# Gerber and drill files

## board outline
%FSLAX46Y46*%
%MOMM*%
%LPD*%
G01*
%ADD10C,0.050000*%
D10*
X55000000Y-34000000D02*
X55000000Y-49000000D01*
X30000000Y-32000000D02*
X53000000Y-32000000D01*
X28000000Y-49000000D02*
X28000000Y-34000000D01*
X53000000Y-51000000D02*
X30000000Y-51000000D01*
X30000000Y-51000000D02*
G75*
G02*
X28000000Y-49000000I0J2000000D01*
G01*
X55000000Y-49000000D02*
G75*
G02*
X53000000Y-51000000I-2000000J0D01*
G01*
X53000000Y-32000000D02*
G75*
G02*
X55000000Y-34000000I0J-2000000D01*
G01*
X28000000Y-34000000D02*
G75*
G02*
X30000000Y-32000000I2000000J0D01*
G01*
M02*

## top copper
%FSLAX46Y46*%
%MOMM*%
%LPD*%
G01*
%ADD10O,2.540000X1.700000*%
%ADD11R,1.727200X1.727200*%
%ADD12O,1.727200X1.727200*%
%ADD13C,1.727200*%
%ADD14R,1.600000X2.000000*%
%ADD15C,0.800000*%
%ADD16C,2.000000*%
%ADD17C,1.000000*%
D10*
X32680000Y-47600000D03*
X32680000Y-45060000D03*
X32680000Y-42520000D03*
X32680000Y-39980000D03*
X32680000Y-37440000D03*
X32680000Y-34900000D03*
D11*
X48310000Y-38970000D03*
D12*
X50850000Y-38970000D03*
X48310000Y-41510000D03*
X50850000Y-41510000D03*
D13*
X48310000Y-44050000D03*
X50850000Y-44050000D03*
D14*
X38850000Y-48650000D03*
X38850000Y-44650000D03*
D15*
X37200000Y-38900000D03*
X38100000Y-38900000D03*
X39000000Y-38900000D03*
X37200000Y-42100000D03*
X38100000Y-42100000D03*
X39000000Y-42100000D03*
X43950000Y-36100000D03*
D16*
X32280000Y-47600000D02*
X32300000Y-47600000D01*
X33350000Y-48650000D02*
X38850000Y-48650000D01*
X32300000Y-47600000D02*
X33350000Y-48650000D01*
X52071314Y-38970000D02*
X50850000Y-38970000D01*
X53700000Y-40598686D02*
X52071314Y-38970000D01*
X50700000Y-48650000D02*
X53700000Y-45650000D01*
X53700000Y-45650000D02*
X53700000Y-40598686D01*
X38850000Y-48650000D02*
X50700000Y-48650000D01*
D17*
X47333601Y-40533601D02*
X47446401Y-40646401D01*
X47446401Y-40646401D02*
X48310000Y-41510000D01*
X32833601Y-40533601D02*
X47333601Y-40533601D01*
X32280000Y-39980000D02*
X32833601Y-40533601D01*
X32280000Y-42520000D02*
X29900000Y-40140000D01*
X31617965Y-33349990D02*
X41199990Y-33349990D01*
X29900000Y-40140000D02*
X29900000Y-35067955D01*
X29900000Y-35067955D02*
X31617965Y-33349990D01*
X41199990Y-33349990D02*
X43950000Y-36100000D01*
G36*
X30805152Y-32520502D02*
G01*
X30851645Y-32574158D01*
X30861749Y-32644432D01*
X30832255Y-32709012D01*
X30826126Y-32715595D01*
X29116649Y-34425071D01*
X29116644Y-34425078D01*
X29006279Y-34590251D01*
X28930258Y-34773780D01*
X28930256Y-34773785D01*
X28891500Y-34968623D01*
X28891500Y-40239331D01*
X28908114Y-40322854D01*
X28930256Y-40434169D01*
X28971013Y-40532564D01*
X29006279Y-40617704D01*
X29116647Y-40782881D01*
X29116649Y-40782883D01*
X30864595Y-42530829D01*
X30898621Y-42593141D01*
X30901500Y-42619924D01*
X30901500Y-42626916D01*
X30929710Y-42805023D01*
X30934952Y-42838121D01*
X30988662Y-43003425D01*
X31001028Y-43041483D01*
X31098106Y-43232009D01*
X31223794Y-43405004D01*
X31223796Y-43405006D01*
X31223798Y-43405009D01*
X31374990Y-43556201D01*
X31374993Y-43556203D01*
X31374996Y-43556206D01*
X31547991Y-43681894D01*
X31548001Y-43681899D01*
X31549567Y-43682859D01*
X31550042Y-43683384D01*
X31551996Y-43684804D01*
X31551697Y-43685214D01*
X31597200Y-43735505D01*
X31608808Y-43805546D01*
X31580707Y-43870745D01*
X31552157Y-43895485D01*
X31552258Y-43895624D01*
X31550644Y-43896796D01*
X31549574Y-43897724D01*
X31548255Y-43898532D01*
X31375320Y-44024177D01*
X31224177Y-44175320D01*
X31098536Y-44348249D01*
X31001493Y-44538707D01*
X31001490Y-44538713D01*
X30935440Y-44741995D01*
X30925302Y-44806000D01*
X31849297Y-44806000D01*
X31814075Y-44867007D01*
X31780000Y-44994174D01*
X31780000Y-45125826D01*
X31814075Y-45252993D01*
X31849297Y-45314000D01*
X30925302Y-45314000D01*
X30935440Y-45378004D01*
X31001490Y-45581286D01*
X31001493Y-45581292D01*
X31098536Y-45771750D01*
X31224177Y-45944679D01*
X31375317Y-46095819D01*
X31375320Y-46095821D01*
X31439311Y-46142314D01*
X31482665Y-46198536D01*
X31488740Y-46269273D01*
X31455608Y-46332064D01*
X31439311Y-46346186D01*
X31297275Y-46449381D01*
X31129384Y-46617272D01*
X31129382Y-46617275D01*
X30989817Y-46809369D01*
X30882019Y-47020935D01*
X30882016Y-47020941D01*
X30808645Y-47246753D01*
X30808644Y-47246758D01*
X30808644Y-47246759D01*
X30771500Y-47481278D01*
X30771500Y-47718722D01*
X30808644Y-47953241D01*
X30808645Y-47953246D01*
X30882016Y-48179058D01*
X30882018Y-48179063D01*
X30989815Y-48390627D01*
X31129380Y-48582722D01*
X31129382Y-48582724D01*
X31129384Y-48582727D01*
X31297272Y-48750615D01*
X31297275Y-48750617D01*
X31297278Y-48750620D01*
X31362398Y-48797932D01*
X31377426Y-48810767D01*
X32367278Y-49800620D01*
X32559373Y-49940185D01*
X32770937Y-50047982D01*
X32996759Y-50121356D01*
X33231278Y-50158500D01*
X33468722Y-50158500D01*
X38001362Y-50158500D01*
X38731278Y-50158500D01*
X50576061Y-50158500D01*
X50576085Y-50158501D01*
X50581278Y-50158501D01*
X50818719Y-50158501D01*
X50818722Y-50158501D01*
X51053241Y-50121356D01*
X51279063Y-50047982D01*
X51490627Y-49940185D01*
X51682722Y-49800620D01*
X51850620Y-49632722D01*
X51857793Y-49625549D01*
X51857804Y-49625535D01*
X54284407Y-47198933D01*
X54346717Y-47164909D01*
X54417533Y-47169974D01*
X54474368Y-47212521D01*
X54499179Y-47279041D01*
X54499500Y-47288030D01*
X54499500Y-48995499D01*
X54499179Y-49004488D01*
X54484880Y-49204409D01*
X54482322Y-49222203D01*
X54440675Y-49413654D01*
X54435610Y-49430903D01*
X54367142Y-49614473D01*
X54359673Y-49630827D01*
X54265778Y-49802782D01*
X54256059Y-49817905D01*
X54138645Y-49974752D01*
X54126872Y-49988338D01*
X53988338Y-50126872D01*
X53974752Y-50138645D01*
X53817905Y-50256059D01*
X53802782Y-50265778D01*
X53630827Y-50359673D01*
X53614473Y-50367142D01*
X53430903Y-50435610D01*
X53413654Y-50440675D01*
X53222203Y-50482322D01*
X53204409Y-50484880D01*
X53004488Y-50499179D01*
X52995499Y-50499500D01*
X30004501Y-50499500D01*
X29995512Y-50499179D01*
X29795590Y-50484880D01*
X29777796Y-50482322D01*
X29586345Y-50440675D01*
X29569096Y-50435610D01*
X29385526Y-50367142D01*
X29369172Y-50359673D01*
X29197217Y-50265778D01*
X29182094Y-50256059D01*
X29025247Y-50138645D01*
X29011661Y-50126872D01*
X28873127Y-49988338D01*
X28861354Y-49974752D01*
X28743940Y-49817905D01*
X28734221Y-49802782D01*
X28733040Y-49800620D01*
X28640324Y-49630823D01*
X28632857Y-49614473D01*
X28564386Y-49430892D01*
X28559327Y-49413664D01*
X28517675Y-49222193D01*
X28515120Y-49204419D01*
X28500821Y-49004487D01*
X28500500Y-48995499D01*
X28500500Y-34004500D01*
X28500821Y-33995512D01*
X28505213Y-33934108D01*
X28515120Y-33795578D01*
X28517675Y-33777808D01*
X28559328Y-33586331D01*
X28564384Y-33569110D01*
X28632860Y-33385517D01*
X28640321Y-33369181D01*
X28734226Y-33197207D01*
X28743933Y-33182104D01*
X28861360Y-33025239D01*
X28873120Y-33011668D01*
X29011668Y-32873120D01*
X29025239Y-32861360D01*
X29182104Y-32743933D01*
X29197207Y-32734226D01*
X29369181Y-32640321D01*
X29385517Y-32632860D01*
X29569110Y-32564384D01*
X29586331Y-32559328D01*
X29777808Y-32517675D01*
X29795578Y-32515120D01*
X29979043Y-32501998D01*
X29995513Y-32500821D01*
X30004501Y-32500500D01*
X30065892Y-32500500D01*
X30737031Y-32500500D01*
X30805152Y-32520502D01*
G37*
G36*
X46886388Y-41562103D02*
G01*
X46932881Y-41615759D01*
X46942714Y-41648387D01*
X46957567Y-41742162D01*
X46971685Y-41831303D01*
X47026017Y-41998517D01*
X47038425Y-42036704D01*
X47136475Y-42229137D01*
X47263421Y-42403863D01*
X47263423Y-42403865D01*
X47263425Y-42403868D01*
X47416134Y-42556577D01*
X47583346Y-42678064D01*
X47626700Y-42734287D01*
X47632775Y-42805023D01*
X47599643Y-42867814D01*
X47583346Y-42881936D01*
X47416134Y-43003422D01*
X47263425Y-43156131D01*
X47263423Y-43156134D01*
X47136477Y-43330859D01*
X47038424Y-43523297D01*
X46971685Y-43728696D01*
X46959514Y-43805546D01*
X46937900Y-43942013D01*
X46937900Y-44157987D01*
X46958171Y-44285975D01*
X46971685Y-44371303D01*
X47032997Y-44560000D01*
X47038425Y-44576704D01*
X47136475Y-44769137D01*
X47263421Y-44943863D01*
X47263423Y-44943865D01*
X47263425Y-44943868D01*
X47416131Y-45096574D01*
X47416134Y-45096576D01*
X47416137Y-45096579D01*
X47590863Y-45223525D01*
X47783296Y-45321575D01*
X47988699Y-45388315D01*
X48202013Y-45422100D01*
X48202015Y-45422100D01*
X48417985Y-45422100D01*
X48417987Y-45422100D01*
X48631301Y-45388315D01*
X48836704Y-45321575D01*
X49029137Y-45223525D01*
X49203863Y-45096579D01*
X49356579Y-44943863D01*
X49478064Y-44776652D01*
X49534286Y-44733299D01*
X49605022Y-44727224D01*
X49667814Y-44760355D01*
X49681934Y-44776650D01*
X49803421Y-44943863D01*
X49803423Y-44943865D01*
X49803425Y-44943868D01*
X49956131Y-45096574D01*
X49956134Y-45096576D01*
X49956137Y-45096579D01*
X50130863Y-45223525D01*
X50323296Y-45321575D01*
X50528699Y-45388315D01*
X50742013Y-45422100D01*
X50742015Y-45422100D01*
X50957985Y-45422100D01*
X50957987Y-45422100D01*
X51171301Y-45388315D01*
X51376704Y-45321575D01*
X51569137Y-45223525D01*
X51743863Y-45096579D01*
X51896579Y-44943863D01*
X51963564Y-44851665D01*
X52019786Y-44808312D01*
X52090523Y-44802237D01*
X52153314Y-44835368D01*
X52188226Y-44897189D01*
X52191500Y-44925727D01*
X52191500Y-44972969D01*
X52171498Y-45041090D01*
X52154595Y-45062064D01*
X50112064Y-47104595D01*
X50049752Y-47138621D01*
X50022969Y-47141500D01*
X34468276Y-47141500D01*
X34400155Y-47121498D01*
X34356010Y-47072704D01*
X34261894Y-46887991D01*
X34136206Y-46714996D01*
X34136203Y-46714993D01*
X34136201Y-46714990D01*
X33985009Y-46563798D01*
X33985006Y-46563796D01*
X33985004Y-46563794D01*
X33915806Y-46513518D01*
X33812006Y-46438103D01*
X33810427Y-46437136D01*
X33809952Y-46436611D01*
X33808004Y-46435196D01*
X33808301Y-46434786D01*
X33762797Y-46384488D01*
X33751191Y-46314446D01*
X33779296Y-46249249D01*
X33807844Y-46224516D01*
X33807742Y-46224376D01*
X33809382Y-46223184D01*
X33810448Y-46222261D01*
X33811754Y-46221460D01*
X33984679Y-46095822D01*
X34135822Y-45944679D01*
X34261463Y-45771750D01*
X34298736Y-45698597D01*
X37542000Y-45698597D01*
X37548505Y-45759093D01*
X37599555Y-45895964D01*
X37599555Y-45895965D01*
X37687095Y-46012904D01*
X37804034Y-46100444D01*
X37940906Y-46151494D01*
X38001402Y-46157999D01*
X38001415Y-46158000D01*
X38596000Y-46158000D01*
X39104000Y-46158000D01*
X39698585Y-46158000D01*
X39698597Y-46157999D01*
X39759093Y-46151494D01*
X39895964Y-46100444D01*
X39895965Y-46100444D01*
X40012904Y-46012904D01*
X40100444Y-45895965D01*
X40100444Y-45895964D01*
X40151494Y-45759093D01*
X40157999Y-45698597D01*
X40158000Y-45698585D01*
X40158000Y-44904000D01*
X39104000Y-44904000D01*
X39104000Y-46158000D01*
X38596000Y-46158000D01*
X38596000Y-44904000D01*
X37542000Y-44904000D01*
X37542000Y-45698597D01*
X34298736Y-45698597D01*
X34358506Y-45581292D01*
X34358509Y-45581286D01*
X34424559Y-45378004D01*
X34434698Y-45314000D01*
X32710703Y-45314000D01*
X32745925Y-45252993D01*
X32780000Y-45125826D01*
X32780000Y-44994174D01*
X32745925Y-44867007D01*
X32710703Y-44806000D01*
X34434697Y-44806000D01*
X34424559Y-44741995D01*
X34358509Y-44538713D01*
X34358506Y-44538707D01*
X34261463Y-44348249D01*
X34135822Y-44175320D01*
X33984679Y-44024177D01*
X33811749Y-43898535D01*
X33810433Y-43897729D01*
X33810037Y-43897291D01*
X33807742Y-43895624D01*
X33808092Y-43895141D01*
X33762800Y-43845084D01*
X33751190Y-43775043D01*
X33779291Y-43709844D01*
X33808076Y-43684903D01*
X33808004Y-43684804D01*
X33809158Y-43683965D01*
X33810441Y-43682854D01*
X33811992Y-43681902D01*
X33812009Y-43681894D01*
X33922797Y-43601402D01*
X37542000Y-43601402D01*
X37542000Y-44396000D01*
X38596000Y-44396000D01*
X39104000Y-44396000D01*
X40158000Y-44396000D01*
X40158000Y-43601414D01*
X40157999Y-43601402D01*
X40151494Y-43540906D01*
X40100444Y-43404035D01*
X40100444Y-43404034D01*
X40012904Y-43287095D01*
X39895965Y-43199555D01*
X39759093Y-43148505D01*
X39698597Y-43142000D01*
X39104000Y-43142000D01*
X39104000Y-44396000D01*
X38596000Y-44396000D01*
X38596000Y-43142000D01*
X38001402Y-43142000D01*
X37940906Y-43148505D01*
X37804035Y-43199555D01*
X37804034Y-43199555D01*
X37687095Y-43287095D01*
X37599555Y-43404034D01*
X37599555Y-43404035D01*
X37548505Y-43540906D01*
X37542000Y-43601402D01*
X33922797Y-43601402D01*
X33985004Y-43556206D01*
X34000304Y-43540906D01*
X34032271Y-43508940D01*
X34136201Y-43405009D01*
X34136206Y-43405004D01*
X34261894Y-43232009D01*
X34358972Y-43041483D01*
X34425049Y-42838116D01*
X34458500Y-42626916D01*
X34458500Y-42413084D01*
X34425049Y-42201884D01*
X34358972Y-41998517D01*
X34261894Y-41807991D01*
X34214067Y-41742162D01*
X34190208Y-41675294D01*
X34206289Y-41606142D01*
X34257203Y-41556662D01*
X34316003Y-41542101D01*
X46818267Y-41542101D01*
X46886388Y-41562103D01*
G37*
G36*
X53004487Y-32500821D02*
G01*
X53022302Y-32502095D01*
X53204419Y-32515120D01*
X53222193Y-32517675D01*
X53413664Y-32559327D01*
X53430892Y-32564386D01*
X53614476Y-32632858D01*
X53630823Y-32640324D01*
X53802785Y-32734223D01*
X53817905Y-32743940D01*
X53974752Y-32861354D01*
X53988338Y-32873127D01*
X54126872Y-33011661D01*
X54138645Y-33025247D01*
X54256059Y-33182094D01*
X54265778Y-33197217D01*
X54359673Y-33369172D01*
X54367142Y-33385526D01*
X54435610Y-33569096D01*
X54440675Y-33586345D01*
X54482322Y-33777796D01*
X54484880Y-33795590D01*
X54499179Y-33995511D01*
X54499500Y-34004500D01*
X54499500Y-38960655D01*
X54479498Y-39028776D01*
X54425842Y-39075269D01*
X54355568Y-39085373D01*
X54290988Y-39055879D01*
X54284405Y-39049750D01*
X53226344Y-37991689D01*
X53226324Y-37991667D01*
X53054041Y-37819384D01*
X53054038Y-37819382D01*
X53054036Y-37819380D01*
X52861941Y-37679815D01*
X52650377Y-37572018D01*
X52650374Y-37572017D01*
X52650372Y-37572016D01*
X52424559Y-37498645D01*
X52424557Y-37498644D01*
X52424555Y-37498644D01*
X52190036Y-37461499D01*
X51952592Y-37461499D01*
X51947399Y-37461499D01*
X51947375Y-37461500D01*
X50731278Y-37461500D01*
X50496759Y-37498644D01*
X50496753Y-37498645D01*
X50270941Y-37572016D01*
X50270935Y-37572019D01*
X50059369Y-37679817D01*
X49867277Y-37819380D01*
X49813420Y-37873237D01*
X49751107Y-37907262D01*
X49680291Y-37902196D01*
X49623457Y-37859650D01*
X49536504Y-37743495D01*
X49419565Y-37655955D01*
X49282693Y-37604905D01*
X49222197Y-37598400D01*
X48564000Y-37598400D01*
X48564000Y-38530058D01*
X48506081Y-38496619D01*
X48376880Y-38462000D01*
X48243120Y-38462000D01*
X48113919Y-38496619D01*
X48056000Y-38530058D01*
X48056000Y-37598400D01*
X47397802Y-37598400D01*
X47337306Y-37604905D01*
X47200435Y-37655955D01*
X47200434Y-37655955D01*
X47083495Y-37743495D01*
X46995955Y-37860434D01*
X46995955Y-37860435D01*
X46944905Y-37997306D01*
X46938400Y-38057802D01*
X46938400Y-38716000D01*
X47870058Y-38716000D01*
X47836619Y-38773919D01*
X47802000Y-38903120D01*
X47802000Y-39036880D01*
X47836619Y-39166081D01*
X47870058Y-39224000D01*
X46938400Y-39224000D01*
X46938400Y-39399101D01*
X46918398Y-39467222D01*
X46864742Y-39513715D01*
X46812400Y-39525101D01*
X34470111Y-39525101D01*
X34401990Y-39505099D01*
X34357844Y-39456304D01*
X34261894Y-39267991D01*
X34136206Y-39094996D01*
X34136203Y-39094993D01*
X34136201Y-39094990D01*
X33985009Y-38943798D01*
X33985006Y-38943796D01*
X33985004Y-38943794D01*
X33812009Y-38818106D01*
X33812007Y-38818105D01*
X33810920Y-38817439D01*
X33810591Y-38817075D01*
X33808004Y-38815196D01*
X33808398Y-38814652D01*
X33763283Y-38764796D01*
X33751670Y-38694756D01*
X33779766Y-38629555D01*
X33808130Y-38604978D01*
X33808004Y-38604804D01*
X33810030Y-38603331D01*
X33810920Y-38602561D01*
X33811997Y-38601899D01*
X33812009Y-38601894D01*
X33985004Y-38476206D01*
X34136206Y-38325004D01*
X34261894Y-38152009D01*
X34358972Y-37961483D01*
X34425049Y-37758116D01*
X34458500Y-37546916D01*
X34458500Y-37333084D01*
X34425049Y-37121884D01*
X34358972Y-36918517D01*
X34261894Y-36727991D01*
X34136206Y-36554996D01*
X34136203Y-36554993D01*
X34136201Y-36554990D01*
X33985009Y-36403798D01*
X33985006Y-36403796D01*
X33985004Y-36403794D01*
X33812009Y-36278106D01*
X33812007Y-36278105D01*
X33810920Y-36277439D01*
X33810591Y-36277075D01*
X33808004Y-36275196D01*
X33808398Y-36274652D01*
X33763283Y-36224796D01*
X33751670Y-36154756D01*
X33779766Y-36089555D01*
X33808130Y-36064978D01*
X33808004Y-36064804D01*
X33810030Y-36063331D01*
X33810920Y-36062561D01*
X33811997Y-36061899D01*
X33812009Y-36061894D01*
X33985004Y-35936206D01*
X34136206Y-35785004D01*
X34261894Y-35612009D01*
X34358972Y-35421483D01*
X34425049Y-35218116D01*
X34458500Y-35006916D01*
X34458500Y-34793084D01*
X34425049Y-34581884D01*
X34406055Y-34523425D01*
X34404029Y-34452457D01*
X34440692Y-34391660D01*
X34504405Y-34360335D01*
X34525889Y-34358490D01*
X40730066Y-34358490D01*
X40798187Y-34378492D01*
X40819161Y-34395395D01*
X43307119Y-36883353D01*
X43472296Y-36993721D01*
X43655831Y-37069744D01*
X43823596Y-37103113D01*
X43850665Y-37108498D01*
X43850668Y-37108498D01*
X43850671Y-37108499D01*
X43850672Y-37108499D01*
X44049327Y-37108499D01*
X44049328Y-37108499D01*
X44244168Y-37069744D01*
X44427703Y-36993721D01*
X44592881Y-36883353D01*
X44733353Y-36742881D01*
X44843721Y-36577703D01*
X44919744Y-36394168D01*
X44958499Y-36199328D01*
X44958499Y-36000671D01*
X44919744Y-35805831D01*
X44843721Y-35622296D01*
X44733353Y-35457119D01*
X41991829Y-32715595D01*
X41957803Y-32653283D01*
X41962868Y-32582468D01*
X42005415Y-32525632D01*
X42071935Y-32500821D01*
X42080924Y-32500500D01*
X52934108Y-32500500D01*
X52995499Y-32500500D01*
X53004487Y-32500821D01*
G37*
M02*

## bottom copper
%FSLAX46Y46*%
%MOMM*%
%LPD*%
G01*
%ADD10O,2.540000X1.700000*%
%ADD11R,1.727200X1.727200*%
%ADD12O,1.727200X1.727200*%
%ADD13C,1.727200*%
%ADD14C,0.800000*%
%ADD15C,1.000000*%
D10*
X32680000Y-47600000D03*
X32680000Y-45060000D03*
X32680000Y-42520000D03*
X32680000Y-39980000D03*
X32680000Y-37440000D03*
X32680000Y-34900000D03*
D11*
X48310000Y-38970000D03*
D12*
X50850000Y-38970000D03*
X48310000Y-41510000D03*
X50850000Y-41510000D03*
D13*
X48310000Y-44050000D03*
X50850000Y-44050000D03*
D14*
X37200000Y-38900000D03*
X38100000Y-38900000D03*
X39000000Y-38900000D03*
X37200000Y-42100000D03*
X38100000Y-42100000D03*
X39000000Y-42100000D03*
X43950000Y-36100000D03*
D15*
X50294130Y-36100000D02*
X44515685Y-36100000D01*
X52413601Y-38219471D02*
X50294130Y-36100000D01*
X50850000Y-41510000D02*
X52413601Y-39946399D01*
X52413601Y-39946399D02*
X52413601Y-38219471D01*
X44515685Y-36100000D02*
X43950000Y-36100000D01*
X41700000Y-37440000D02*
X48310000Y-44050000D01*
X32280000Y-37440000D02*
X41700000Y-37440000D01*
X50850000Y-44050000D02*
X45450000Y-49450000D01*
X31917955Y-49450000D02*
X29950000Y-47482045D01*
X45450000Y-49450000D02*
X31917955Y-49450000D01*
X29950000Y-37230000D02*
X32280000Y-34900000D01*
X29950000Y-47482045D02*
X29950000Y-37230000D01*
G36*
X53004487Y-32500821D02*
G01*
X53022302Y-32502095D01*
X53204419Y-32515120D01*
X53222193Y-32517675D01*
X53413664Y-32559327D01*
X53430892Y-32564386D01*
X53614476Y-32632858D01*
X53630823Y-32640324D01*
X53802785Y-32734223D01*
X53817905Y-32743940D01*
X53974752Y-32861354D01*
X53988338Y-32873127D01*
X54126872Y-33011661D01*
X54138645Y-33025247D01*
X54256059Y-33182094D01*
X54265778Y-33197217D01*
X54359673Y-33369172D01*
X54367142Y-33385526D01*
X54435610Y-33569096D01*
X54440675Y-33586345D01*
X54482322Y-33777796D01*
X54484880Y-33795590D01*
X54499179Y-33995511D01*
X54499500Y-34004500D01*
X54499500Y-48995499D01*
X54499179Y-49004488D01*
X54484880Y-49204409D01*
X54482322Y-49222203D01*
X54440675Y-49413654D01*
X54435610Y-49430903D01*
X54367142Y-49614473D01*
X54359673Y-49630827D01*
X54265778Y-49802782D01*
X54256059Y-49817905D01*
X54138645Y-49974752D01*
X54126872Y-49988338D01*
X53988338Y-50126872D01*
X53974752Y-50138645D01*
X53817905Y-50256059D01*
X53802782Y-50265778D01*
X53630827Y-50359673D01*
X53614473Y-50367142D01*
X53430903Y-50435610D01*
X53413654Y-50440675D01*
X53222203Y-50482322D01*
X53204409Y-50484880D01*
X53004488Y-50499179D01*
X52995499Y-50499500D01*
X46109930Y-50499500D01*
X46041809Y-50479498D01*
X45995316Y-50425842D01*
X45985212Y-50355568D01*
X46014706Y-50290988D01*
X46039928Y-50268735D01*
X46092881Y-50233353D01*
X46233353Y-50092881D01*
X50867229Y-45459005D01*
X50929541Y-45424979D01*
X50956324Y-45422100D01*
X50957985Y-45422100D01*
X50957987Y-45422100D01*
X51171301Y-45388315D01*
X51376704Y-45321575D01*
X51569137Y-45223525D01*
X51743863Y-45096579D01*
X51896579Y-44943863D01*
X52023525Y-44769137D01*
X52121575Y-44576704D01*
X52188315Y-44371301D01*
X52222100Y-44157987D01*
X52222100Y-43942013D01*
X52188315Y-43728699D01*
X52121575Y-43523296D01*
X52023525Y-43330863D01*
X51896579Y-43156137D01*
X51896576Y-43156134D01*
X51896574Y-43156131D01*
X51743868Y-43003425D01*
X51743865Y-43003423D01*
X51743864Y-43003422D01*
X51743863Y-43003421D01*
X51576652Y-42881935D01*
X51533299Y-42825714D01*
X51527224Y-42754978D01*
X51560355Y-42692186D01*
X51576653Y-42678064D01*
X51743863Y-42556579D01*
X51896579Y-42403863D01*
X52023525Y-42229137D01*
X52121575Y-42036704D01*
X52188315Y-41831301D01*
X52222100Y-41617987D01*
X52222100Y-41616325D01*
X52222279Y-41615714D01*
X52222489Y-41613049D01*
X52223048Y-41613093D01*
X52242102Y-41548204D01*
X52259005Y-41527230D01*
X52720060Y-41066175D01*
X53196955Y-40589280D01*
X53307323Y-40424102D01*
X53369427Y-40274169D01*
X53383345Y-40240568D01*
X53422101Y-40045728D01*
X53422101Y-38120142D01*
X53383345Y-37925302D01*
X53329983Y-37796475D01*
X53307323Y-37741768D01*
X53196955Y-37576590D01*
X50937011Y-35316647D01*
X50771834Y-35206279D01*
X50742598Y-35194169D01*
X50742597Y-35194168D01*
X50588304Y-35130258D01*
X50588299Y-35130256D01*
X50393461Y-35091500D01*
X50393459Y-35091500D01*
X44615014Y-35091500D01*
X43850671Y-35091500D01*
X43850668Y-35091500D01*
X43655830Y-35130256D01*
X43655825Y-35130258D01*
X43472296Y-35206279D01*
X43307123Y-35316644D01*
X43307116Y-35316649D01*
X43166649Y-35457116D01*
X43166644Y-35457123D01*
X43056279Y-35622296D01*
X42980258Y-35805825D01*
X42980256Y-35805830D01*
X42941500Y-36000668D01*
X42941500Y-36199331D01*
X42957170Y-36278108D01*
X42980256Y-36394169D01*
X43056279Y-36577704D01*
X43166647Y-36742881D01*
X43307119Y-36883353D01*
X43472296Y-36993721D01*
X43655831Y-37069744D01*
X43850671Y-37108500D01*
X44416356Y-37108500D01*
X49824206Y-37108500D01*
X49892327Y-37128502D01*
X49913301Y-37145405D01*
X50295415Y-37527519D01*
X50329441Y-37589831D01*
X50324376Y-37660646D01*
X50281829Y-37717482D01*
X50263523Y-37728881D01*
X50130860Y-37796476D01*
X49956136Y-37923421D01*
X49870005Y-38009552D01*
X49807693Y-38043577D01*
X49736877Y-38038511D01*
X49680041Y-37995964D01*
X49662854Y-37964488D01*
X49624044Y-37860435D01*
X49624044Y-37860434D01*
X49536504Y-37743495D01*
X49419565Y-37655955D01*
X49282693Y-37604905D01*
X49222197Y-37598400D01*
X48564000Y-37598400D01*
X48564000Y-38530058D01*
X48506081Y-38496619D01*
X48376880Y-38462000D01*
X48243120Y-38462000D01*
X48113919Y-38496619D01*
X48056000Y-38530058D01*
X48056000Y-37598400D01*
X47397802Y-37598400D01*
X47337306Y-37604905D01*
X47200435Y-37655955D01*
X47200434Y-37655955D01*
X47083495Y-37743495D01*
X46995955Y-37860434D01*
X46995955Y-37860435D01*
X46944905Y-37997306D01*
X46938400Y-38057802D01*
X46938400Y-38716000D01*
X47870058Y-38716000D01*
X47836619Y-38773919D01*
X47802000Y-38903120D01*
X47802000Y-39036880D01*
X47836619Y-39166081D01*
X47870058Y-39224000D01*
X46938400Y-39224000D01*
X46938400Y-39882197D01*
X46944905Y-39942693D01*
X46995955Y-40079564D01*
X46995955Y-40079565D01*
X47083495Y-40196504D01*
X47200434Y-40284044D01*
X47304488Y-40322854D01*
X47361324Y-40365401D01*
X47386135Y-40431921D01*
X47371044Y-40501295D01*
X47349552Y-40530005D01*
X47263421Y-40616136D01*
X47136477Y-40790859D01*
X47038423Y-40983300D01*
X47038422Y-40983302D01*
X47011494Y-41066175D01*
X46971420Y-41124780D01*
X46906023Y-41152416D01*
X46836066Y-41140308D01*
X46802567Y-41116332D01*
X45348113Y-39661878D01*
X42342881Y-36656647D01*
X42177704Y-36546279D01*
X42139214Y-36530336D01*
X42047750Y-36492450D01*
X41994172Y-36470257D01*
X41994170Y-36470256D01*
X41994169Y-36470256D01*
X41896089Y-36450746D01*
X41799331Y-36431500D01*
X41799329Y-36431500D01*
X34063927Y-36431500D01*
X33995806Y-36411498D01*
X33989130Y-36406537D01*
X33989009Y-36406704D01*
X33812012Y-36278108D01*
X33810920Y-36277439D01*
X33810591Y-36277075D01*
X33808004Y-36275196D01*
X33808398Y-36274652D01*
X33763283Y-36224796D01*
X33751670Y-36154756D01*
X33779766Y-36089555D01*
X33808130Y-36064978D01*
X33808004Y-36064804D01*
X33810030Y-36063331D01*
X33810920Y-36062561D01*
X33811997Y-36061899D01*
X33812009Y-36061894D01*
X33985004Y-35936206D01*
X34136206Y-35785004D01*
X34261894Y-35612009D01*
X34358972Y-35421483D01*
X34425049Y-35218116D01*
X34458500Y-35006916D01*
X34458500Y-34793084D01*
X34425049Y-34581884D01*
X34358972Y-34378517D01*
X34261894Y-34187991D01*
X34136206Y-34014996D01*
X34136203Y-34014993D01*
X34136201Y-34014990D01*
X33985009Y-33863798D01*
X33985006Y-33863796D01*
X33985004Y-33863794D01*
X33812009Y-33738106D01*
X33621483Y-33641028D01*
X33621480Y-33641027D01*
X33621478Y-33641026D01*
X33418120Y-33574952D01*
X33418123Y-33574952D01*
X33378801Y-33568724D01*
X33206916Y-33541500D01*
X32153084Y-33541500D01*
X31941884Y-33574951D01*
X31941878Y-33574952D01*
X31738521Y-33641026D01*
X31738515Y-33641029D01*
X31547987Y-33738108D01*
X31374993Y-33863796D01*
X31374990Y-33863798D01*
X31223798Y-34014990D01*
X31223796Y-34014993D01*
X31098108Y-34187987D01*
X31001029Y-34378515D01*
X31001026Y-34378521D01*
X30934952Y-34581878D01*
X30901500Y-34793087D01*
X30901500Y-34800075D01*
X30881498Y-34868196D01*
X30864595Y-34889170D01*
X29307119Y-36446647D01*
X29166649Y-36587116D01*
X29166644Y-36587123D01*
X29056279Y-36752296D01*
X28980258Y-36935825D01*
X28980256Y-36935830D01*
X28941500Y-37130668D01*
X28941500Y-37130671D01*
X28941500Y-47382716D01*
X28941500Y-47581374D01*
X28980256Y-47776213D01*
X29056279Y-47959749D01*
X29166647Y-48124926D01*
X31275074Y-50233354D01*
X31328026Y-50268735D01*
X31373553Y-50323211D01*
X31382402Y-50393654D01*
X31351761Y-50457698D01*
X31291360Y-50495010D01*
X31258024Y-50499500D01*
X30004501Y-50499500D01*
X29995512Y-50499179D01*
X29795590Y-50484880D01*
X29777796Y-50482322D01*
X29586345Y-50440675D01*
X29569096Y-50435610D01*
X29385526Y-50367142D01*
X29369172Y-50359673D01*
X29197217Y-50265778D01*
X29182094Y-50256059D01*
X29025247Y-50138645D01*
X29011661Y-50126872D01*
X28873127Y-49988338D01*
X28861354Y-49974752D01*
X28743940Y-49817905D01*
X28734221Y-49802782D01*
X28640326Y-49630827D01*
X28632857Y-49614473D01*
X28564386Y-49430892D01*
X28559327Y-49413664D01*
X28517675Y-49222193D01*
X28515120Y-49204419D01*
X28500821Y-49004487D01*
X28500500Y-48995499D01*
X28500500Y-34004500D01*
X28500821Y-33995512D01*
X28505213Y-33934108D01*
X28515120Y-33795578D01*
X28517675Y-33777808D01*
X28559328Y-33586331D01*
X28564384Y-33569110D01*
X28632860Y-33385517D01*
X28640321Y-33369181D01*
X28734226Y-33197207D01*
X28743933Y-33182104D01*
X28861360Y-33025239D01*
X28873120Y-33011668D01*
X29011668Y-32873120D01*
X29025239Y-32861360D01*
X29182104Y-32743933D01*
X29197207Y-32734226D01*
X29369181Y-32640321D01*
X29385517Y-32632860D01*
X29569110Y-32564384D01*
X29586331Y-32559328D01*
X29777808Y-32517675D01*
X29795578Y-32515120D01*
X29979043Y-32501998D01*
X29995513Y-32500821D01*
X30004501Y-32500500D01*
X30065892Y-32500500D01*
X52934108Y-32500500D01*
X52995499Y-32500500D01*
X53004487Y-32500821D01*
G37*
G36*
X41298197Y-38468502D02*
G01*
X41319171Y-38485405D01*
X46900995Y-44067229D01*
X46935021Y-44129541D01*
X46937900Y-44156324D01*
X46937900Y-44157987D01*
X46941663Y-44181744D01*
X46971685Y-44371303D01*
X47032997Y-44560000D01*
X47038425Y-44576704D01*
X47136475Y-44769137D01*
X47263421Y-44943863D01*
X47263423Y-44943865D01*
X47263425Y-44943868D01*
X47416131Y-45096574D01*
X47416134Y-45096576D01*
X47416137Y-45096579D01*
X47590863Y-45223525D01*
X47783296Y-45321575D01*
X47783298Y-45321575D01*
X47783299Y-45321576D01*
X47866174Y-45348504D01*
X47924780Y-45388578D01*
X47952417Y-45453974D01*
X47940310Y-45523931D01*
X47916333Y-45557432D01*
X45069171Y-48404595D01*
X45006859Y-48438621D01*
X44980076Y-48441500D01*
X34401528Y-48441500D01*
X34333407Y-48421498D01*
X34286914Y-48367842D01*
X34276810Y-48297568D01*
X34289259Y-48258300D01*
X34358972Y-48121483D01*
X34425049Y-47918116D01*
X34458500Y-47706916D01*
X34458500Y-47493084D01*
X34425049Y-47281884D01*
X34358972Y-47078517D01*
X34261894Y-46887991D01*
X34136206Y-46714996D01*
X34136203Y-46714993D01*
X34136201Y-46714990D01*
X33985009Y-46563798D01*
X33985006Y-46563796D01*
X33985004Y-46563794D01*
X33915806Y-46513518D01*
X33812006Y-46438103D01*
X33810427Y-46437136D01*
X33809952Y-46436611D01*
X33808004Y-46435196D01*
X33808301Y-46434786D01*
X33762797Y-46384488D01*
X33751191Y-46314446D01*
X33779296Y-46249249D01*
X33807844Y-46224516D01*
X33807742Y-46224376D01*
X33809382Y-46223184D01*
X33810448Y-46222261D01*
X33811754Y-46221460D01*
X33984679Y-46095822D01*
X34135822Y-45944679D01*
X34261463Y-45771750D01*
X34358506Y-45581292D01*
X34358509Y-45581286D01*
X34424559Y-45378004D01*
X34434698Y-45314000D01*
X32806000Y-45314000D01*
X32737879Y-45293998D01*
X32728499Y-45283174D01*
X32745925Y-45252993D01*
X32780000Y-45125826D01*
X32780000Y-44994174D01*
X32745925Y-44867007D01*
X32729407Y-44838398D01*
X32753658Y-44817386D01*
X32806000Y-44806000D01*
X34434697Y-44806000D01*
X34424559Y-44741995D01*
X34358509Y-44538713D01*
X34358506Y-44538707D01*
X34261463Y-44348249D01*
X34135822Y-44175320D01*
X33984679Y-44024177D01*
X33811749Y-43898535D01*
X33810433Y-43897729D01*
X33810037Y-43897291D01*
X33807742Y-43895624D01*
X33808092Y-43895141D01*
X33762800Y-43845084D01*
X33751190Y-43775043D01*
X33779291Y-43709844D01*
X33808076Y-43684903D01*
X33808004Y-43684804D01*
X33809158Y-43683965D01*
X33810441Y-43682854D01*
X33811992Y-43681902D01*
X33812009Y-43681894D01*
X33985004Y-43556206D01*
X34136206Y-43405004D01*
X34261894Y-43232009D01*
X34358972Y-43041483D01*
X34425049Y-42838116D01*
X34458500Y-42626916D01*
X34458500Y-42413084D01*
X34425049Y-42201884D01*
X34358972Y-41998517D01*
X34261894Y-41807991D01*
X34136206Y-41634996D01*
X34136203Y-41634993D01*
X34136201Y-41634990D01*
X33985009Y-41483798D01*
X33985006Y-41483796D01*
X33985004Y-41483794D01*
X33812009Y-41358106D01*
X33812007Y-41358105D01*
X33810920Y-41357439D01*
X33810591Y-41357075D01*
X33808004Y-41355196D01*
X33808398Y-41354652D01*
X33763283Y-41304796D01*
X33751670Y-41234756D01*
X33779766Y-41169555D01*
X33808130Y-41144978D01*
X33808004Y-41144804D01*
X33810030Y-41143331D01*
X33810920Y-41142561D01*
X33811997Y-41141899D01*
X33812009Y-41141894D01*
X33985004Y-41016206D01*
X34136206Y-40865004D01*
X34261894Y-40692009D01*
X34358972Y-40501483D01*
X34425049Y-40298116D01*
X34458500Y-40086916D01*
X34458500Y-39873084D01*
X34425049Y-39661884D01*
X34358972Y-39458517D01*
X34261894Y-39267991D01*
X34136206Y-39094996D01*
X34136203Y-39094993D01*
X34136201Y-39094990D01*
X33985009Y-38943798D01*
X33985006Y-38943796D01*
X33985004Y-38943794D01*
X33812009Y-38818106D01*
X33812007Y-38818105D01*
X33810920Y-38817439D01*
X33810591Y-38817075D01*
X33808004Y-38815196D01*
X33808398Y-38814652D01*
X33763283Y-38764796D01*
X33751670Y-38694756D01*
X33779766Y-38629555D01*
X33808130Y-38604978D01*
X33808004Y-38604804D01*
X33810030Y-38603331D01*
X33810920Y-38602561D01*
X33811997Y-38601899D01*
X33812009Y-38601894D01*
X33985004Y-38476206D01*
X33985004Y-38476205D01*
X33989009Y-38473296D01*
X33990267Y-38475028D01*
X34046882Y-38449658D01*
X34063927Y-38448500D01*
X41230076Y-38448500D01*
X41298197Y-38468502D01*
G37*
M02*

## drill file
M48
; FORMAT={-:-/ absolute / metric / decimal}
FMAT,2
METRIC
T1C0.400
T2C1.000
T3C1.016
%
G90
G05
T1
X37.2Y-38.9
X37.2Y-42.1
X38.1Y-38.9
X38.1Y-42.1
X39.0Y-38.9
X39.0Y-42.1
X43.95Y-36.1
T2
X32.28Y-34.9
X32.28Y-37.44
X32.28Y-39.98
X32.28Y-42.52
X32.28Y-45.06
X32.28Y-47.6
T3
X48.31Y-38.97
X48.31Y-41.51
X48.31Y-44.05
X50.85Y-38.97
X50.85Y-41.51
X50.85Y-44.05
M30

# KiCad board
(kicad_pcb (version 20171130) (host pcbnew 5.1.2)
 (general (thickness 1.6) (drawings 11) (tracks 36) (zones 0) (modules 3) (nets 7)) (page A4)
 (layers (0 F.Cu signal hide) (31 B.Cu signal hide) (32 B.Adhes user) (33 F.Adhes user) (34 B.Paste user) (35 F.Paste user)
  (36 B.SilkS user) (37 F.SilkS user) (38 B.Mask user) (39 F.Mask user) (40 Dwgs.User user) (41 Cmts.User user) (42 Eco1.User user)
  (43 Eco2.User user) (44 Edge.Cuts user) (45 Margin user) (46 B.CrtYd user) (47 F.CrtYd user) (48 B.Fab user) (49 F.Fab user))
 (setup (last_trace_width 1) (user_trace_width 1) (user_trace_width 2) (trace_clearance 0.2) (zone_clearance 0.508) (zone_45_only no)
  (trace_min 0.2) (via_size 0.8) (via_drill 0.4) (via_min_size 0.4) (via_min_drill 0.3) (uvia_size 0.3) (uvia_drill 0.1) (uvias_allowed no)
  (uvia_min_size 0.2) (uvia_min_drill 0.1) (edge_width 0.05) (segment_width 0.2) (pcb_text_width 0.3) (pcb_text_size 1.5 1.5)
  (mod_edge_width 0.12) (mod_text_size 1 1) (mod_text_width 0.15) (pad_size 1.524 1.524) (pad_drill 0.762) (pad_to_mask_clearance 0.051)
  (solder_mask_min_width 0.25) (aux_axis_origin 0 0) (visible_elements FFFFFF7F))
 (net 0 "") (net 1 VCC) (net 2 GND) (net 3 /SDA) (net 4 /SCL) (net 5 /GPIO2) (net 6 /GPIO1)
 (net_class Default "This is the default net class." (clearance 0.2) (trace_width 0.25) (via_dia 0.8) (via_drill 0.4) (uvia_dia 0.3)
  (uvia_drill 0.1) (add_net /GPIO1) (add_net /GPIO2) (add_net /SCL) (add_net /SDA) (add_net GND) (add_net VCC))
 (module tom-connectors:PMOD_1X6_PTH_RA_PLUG (layer F.Cu) (at 33.55 41.25 270)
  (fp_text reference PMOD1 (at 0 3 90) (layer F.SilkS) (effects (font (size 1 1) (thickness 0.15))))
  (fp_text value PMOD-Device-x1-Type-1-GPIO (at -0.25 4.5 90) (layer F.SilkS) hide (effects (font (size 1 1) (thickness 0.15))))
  (pad 6 thru_hole oval (at 6.35 1.27 180) (size 2.54 1.7) (drill 1 (offset -0.4 0)) (layers *.Cu *.Mask) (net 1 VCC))
  (pad 5 thru_hole oval (at 3.81 1.27 180) (size 2.54 1.7) (drill 1 (offset -0.4 0)) (layers *.Cu *.Mask) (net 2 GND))
  (pad 4 thru_hole oval (at 1.27 1.27 180) (size 2.54 1.7) (drill 1 (offset -0.4 0)) (layers *.Cu *.Mask) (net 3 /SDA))
  (pad 3 thru_hole oval (at -1.27 1.27 180) (size 2.54 1.7) (drill 1 (offset -0.4 0)) (layers *.Cu *.Mask) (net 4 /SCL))
  (pad 2 thru_hole oval (at -3.81 1.27 180) (size 2.54 1.7) (drill 1 (offset -0.4 0)) (layers *.Cu *.Mask) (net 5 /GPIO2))
  (pad 1 thru_hole oval (at -6.35 1.27 180) (size 2.54 1.7) (drill 1 (offset -0.4 0)) (layers *.Cu *.Mask) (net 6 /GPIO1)))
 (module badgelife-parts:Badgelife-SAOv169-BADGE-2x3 (layer F.Cu) (at 49.6 41.45 270)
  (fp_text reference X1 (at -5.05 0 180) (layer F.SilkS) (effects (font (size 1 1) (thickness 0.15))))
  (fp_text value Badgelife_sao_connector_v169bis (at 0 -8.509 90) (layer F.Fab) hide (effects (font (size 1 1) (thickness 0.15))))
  (pad 2 thru_hole rect (at -2.48 1.29 180) (size 1.7272 1.7272) (drill 1.016) (layers *.Cu *.Mask) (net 2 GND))
  (pad 1 thru_hole oval (at -2.48 -1.25 180) (size 1.7272 1.7272) (drill 1.016) (layers *.Cu *.Mask) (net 1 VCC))
  (pad 4 thru_hole oval (at 0.06 1.29 180) (size 1.7272 1.7272) (drill 1.016) (layers *.Cu *.Mask) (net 4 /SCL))
  (pad 3 thru_hole oval (at 0.06 -1.25 180) (size 1.7272 1.7272) (drill 1.016) (layers *.Cu *.Mask) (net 3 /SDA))
  (pad 6 thru_hole circle (at 2.6 1.29 180) (size 1.7272 1.7272) (drill 1.016) (layers *.Cu *.Mask) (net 5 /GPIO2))
  (pad 5 thru_hole circle (at 2.6 -1.25 180) (size 1.7272 1.7272) (drill 1.016) (layers *.Cu *.Mask) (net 6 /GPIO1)))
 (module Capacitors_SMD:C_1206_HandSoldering (layer F.Cu) (at 38.85 46.65 90)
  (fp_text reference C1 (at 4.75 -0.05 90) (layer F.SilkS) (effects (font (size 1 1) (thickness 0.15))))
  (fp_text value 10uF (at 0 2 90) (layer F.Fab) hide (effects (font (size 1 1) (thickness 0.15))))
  (pad 1 smd rect (at -2 0 90) (size 2 1.6) (layers F.Cu F.Paste F.Mask) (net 1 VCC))
  (pad 2 smd rect (at 2 0 90) (size 2 1.6) (layers F.Cu F.Paste F.Mask) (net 2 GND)))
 (gr_line (start 55 34) (end 55 49) (layer Edge.Cuts) (width 0.05))
 (gr_line (start 30 32) (end 53 32) (layer Edge.Cuts) (width 0.05))
 (gr_line (start 28 49) (end 28 34) (layer Edge.Cuts) (width 0.05))
 (gr_line (start 53 51) (end 30 51) (layer Edge.Cuts) (width 0.05))
 (gr_arc (start 30 49) (end 28 49) (angle -90) (layer Edge.Cuts) (width 0.05))
 (gr_arc (start 53 49) (end 53 51) (angle -90) (layer Edge.Cuts) (width 0.05))
 (gr_arc (start 53 34) (end 55 34) (angle -90) (layer Edge.Cuts) (width 0.05))
 (gr_arc (start 30 34) (end 30 32) (angle -90) (layer Edge.Cuts) (width 0.05))
 (segment (start 32.28 47.6) (end 32.3 47.6) (width 2) (layer F.Cu) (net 1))
 (segment (start 33.35 48.65) (end 38.85 48.65) (width 2) (layer F.Cu) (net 1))
 (segment (start 32.3 47.6) (end 33.35 48.65) (width 2) (layer F.Cu) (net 1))
 (segment (start 52.071314 38.97) (end 50.85 38.97) (width 2) (layer F.Cu) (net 1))
 (segment (start 53.7 40.598686) (end 52.071314 38.97) (width 2) (layer F.Cu) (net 1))
 (segment (start 50.7 48.65) (end 53.7 45.65) (width 2) (layer F.Cu) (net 1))
 (segment (start 53.7 45.65) (end 53.7 40.598686) (width 2) (layer F.Cu) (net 1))
 (segment (start 38.85 48.65) (end 50.7 48.65) (width 2) (layer F.Cu) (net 1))
 (via (at 37.2 38.9) (size 0.8) (drill 0.4) (layers F.Cu B.Cu) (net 2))
 (via (at 38.1 38.9) (size 0.8) (drill 0.4) (layers F.Cu B.Cu) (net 2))
 (via (at 39 38.9) (size 0.8) (drill 0.4) (layers F.Cu B.Cu) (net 2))
 (via (at 37.2 42.1) (size 0.8) (drill 0.4) (layers F.Cu B.Cu) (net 2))
 (via (at 38.1 42.1) (size 0.8) (drill 0.4) (layers F.Cu B.Cu) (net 2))
 (via (at 39 42.1) (size 0.8) (drill 0.4) (layers F.Cu B.Cu) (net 2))
 (segment (start 47.333601 40.533601) (end 47.446401 40.646401) (width 1) (layer F.Cu) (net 4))
 (segment (start 47.446401 40.646401) (end 48.31 41.51) (width 1) (layer F.Cu) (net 4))
 (segment (start 32.833601 40.533601) (end 47.333601 40.533601) (width 1) (layer F.Cu) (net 4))
 (segment (start 32.28 39.98) (end 32.833601 40.533601) (width 1) (layer F.Cu) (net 4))
 (segment (start 32.28 42.52) (end 29.9 40.14) (width 1) (layer F.Cu) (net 3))
 (segment (start 31.617965 33.34999) (end 41.19999 33.34999) (width 1) (layer F.Cu) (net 3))
 (segment (start 29.9 40.14) (end 29.9 35.067955) (width 1) (layer F.Cu) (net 3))
 (segment (start 29.9 35.067955) (end 31.617965 33.34999) (width 1) (layer F.Cu) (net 3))
 (segment (start 41.19999 33.34999) (end 43.95 36.1) (width 1) (layer F.Cu) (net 3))
 (via (at 43.95 36.1) (size 0.8) (drill 0.4) (layers F.Cu B.Cu) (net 3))
 (segment (start 50.29413 36.1) (end 44.515685 36.1) (width 1) (layer B.Cu) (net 3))
 (segment (start 52.413601 38.219471) (end 50.29413 36.1) (width 1) (layer B.Cu) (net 3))
 (segment (start 50.85 41.51) (end 52.413601 39.946399) (width 1) (layer B.Cu) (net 3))
 (segment (start 52.413601 39.946399) (end 52.413601 38.219471) (width 1) (layer B.Cu) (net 3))
 (segment (start 44.515685 36.1) (end 43.95 36.1) (width 1) (layer B.Cu) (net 3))
 (segment (start 41.7 37.44) (end 48.31 44.05) (width 1) (layer B.Cu) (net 5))
 (segment (start 32.28 37.44) (end 41.7 37.44) (width 1) (layer B.Cu) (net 5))
 (segment (start 50.85 44.05) (end 45.45 49.45) (width 1) (layer B.Cu) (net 6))
 (segment (start 31.917955 49.45) (end 29.95 47.482045) (width 1) (layer B.Cu) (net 6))
 (segment (start 45.45 49.45) (end 31.917955 49.45) (width 1) (layer B.Cu) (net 6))
 (segment (start 29.95 37.23) (end 32.28 34.9) (width 1) (layer B.Cu) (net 6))
 (segment (start 29.95 47.482045) (end 29.95 37.23) (width 1) (layer B.Cu) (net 6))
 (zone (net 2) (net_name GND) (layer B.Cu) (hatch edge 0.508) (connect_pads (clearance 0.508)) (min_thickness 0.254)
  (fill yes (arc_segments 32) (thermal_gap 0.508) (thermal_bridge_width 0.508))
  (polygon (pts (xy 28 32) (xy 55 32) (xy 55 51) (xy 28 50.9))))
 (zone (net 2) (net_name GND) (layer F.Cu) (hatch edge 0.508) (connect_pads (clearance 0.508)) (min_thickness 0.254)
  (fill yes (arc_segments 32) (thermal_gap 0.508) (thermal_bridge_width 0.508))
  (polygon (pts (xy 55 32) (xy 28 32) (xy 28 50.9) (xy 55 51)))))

